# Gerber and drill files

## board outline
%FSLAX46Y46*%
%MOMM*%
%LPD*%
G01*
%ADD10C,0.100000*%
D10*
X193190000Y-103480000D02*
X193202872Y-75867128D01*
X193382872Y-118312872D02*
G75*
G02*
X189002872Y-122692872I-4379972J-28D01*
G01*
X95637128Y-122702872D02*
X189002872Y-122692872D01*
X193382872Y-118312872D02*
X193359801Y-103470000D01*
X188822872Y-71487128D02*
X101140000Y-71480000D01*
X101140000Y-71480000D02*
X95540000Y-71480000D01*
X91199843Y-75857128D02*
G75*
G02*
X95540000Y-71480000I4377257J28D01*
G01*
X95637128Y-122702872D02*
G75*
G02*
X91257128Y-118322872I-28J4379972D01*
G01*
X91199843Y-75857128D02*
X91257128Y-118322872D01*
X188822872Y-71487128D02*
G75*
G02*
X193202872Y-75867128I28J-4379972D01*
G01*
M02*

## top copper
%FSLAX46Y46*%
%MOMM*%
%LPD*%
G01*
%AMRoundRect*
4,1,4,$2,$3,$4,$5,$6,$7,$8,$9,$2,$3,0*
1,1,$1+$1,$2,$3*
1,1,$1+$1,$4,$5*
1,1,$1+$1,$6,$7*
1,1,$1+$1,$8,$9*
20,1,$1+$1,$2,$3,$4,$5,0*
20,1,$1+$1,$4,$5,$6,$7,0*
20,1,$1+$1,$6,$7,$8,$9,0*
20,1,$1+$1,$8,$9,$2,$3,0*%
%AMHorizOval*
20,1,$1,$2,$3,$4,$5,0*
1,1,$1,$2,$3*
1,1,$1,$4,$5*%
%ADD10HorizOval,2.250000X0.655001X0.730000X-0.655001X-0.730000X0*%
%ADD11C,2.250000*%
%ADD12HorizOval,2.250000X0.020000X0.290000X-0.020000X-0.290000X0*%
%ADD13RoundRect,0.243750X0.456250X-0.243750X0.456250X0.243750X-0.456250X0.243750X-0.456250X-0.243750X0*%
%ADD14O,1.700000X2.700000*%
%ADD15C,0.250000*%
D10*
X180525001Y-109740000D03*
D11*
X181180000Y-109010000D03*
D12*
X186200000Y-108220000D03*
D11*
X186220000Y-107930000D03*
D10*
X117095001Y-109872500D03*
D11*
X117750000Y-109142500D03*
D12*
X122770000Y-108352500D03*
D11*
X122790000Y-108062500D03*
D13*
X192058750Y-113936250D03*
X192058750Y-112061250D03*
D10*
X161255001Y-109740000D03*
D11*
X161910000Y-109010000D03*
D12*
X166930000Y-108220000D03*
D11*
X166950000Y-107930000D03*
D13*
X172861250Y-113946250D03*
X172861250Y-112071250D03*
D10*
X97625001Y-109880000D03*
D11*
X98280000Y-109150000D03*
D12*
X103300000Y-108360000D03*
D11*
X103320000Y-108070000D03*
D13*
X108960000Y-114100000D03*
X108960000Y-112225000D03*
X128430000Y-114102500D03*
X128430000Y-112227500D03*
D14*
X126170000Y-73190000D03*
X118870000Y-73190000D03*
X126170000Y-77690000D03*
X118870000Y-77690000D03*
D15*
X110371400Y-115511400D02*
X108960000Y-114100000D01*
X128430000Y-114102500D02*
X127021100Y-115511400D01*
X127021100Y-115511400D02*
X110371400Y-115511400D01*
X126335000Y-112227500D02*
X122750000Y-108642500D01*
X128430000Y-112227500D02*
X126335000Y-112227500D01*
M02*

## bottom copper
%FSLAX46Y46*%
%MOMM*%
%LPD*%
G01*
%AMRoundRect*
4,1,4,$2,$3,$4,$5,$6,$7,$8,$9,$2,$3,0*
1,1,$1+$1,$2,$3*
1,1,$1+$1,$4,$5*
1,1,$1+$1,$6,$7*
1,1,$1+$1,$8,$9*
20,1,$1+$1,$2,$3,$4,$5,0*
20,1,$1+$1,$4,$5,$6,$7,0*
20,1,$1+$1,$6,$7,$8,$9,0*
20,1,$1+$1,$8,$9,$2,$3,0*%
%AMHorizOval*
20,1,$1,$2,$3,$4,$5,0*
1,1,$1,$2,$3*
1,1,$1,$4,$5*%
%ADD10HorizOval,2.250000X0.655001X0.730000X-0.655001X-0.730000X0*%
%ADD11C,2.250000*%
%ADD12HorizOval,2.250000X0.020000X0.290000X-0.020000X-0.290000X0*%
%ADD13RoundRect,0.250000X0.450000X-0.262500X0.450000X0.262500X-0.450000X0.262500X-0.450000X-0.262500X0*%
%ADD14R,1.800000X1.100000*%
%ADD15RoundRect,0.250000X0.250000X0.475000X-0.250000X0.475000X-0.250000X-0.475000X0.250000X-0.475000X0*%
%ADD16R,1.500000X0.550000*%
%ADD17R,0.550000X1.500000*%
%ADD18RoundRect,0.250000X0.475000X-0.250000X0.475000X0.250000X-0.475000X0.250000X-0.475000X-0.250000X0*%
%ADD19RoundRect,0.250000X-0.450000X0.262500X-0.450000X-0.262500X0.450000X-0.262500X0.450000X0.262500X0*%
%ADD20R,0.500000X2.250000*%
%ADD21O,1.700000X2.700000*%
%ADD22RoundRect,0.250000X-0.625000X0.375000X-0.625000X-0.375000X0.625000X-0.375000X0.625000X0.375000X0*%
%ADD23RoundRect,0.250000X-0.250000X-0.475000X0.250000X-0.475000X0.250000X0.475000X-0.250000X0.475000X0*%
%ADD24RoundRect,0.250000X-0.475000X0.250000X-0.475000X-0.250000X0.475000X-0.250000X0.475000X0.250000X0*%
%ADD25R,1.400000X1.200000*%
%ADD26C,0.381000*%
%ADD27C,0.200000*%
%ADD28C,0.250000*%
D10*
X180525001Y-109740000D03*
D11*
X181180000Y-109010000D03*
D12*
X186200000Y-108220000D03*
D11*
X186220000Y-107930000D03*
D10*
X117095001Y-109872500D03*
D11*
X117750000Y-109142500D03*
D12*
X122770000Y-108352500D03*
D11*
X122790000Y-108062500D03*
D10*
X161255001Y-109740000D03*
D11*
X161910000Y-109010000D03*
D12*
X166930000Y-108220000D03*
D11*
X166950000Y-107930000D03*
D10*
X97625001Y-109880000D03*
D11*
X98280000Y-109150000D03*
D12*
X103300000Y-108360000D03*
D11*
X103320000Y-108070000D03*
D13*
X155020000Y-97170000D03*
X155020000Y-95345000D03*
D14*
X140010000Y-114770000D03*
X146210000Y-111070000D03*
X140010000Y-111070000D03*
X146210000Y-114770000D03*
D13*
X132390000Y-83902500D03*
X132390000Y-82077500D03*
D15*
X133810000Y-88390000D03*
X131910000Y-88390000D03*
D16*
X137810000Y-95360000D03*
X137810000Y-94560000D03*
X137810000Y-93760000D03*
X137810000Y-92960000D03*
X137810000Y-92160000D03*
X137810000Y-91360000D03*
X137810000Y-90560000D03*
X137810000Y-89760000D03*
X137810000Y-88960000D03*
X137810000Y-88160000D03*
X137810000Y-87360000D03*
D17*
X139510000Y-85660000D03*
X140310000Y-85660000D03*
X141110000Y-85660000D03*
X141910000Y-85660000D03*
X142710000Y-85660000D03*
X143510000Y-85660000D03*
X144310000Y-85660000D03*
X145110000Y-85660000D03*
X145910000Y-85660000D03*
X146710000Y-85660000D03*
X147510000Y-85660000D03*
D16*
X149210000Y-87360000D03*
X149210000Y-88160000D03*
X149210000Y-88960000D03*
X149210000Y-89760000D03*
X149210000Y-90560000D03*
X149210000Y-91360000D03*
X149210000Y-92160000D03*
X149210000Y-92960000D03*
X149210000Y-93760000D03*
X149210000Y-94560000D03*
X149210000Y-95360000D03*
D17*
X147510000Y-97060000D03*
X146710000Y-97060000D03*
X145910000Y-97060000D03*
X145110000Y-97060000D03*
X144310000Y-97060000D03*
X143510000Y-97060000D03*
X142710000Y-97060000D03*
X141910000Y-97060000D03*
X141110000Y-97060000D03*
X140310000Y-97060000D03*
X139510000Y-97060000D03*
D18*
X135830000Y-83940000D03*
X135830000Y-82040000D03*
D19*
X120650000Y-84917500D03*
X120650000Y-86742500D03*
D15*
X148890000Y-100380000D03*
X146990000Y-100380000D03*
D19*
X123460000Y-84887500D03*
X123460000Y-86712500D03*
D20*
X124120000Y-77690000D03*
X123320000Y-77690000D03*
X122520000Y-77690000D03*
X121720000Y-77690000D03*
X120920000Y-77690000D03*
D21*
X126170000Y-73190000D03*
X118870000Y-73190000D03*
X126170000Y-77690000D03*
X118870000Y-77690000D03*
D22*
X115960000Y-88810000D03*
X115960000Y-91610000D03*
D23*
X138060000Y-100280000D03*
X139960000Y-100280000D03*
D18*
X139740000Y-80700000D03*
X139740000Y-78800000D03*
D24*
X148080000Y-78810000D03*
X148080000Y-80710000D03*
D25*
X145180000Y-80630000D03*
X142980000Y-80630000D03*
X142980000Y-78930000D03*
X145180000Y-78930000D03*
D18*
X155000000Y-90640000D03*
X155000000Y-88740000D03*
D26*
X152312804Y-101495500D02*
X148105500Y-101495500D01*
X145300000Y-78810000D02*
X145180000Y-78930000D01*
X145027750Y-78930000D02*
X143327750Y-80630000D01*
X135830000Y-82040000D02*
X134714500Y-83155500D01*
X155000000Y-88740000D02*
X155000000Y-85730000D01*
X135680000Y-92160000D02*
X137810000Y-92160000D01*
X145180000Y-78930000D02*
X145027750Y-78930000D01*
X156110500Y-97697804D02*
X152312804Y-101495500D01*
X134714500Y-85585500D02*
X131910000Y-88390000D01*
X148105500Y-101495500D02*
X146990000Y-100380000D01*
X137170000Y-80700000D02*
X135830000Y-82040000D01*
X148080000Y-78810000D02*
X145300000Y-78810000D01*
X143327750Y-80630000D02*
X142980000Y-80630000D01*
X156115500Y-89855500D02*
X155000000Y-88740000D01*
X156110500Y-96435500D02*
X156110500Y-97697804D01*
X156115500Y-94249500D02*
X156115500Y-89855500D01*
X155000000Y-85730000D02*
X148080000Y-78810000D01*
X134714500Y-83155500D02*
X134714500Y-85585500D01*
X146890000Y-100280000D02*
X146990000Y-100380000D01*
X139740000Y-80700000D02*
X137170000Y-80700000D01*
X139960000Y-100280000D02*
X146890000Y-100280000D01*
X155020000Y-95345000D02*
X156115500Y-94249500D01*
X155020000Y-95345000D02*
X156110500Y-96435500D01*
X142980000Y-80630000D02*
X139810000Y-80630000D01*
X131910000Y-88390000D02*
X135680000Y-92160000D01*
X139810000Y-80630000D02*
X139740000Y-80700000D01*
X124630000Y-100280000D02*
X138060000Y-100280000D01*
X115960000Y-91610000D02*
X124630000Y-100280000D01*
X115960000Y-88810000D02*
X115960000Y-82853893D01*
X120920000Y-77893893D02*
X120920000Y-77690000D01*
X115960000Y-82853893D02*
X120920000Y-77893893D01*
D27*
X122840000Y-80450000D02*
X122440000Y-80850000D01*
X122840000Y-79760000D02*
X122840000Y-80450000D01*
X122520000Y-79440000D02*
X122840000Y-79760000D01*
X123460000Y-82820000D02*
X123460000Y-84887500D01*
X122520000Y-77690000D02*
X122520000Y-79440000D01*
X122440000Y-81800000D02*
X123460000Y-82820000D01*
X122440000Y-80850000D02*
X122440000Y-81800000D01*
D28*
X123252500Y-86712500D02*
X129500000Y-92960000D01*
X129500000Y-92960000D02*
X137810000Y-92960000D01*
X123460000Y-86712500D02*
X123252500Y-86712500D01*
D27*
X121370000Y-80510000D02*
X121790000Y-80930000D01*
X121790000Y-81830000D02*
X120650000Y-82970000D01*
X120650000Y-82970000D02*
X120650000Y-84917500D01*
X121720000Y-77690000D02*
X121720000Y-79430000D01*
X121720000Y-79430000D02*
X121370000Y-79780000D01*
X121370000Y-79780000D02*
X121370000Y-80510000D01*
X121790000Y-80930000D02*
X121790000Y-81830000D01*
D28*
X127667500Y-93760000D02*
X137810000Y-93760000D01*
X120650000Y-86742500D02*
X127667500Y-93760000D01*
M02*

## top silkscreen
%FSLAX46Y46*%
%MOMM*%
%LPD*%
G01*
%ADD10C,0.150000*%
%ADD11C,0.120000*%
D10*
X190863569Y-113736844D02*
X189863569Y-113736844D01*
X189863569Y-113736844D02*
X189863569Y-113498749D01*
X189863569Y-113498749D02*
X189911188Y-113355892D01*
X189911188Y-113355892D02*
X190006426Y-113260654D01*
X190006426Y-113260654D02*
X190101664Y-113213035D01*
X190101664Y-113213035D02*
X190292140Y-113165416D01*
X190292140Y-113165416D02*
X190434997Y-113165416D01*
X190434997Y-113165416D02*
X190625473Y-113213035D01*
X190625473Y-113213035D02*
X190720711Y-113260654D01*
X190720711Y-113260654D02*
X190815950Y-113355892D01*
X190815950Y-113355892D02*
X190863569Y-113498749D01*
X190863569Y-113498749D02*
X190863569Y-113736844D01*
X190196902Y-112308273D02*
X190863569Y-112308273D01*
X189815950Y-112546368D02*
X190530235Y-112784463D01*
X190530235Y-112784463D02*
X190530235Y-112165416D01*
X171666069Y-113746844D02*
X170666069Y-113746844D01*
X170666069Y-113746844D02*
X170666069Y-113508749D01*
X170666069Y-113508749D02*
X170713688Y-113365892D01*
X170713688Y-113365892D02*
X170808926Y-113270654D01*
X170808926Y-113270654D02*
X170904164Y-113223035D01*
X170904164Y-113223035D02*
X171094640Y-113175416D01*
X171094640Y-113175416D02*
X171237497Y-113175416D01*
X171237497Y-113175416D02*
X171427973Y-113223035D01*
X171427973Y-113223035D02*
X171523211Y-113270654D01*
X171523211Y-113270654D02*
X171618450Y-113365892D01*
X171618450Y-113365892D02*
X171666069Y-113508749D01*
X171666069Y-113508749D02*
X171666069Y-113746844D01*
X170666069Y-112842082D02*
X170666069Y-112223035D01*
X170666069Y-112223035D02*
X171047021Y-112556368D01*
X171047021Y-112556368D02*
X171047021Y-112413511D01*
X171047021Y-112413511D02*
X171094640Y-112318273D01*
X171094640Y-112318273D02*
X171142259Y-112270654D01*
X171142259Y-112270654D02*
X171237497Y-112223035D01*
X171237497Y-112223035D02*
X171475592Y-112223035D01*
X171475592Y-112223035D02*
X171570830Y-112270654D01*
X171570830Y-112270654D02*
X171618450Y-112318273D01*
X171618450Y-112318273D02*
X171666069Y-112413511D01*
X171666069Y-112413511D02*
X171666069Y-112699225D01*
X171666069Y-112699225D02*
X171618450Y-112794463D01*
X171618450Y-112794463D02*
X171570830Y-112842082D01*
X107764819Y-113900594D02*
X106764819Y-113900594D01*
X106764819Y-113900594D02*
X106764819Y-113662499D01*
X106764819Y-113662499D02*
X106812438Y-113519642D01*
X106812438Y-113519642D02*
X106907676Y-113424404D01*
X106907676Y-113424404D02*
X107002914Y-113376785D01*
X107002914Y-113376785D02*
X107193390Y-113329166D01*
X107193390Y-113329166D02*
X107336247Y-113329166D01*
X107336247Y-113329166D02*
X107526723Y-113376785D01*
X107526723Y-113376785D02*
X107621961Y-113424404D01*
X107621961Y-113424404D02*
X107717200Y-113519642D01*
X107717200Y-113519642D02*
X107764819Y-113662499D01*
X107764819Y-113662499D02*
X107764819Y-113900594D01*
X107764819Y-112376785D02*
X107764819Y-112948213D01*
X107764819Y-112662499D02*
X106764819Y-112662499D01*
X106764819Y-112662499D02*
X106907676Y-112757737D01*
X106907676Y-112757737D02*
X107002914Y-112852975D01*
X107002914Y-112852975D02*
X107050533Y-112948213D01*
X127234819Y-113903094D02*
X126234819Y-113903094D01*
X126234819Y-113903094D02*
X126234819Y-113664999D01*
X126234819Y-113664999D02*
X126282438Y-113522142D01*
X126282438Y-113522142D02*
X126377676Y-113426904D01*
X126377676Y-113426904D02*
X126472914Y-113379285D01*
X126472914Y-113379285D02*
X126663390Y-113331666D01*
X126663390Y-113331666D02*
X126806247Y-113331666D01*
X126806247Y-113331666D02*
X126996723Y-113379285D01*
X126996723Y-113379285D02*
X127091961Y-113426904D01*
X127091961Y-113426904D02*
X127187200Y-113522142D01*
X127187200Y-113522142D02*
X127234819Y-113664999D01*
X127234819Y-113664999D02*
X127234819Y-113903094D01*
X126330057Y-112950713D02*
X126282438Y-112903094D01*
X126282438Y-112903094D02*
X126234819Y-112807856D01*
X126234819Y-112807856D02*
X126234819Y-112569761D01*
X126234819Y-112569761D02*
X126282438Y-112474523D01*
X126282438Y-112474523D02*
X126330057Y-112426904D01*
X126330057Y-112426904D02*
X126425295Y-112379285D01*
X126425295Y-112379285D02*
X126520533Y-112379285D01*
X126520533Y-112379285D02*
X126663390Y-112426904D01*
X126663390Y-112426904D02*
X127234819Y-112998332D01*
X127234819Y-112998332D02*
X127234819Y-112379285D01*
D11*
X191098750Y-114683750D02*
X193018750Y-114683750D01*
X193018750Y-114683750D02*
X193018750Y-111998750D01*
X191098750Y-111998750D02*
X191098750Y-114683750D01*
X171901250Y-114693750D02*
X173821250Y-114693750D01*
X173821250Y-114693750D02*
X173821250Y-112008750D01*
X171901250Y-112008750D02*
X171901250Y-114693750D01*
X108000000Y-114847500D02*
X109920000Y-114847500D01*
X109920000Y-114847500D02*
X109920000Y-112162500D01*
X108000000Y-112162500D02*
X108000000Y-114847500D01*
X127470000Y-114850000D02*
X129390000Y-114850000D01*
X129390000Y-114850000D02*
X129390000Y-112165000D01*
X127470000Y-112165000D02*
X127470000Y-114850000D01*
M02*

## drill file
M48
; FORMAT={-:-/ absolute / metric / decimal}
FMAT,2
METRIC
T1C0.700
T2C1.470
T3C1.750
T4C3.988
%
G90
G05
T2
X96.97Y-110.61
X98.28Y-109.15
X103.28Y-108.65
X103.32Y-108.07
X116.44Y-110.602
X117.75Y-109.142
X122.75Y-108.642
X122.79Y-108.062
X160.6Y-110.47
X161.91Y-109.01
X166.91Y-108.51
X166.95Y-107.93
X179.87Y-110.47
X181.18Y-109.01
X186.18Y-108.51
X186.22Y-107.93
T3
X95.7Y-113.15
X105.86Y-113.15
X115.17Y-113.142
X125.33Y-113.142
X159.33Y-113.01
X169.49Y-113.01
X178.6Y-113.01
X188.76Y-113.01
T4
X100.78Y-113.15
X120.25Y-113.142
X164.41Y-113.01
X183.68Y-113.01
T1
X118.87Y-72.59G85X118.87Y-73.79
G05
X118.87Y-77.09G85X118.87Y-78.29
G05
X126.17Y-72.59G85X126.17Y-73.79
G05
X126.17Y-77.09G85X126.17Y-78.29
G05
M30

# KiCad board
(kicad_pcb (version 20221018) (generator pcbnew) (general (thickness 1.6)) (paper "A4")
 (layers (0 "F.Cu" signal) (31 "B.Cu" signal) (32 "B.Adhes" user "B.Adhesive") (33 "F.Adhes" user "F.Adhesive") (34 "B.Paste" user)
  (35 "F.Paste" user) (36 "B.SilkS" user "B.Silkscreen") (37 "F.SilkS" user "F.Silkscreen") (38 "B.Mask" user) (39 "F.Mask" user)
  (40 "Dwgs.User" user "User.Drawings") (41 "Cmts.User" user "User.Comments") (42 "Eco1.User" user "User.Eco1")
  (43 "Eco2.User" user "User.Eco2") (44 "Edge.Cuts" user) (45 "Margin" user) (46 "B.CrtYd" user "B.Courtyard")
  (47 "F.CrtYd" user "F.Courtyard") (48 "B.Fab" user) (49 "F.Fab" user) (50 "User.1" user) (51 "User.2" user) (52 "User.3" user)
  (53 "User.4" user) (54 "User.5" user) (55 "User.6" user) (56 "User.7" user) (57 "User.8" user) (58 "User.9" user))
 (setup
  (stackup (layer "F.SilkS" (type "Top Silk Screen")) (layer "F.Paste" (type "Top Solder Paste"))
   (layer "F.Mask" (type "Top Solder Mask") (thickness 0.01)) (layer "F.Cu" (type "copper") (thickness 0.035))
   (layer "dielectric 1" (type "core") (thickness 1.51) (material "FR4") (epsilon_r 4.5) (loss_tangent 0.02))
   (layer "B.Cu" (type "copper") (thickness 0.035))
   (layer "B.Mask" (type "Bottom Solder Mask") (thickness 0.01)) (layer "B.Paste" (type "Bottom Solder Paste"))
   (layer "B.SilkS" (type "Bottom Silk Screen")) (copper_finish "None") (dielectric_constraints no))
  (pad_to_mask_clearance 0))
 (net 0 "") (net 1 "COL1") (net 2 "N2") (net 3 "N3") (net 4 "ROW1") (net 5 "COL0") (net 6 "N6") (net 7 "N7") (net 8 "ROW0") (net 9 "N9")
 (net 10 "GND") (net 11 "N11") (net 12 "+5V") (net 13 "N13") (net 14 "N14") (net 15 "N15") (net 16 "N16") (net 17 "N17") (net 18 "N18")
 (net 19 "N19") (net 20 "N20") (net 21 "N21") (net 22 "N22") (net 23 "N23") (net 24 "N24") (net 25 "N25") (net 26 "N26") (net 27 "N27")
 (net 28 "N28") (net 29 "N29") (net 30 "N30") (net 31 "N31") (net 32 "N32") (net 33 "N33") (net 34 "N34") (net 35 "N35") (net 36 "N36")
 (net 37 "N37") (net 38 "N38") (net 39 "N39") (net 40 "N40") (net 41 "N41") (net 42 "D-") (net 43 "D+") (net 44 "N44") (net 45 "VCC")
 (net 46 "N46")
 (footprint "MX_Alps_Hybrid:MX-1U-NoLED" (layer "F.Cu") (at 183.68 113.01)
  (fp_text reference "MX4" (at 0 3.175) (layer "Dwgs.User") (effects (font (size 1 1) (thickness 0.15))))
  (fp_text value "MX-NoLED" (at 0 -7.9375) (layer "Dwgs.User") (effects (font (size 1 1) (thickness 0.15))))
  (pad "" np_thru_hole circle (at -5.08 0 48.0996) (size 1.75 1.75) (drill 1.75) (layers "*.Cu" "*.Mask"))
  (pad "" np_thru_hole circle (at 0 0) (size 3.9878 3.9878) (drill 3.9878) (layers "*.Cu" "*.Mask"))
  (pad "" np_thru_hole circle (at 5.08 0 48.0996) (size 1.75 1.75) (drill 1.75) (layers "*.Cu" "*.Mask"))
  (pad "1" thru_hole oval (at -3.81 -2.54 48.0996) (size 4.211556 2.25) (drill 1.47 (offset 0.980778 0)) (layers "*.Cu" "B.Mask")
   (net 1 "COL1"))
  (pad "1" thru_hole circle (at -2.5 -4) (size 2.25 2.25) (drill 1.47) (layers "*.Cu" "B.Mask") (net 1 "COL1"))
  (pad "2" thru_hole oval (at 2.5 -4.5 86.0548) (size 2.831378 2.25) (drill 1.47 (offset 0.290689 0)) (layers "*.Cu" "B.Mask") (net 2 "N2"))
  (pad "2" thru_hole circle (at 2.54 -5.08) (size 2.25 2.25) (drill 1.47) (layers "*.Cu" "B.Mask") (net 2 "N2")))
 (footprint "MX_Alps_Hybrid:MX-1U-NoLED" (layer "F.Cu") (at 120.25 113.1425)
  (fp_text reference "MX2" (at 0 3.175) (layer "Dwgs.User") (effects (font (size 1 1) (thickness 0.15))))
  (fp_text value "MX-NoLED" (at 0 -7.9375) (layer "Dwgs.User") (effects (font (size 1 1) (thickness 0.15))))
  (pad "" np_thru_hole circle (at -5.08 0 48.0996) (size 1.75 1.75) (drill 1.75) (layers "*.Cu" "*.Mask"))
  (pad "" np_thru_hole circle (at 0 0) (size 3.9878 3.9878) (drill 3.9878) (layers "*.Cu" "*.Mask"))
  (pad "" np_thru_hole circle (at 5.08 0 48.0996) (size 1.75 1.75) (drill 1.75) (layers "*.Cu" "*.Mask"))
  (pad "1" thru_hole oval (at -3.81 -2.54 48.0996) (size 4.211556 2.25) (drill 1.47 (offset 0.980778 0)) (layers "*.Cu" "B.Mask")
   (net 1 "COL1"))
  (pad "1" thru_hole circle (at -2.5 -4) (size 2.25 2.25) (drill 1.47) (layers "*.Cu" "B.Mask") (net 1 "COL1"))
  (pad "2" thru_hole oval (at 2.5 -4.5 86.0548) (size 2.831378 2.25) (drill 1.47 (offset 0.290689 0)) (layers "*.Cu" "B.Mask") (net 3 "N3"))
  (pad "2" thru_hole circle (at 2.54 -5.08) (size 2.25 2.25) (drill 1.47) (layers "*.Cu" "B.Mask") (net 3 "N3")))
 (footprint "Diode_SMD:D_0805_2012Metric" (layer "F.Cu") (at 192.05875 112.99875 90)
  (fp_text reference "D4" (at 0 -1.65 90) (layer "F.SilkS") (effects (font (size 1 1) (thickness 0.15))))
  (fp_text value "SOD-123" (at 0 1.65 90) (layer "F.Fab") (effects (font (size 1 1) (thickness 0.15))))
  (fp_line (start -1.685 -0.96) (end -1.685 0.96) (stroke (width 0.12) (type solid)) (layer "F.SilkS"))
  (fp_line (start -1.685 0.96) (end 1 0.96) (stroke (width 0.12) (type solid)) (layer "F.SilkS"))
  (fp_line (start 1 -0.96) (end -1.685 -0.96) (stroke (width 0.12) (type solid)) (layer "F.SilkS"))
  (pad "1" smd roundrect (at -0.9375 0 90) (size 0.975 1.4) (layers "F.Cu" "F.Paste" "F.Mask") (roundrect_rratio 0.25) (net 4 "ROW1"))
  (pad "2" smd roundrect (at 0.9375 0 90) (size 0.975 1.4) (layers "F.Cu" "F.Paste" "F.Mask") (roundrect_rratio 0.25) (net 2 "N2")))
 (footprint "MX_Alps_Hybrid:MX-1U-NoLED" (layer "F.Cu") (at 164.41 113.01)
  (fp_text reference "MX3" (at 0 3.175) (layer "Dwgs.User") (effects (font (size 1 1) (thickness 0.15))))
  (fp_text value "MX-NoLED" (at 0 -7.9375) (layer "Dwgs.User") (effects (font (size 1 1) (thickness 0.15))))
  (pad "" np_thru_hole circle (at -5.08 0 48.0996) (size 1.75 1.75) (drill 1.75) (layers "*.Cu" "*.Mask"))
  (pad "" np_thru_hole circle (at 0 0) (size 3.9878 3.9878) (drill 3.9878) (layers "*.Cu" "*.Mask"))
  (pad "" np_thru_hole circle (at 5.08 0 48.0996) (size 1.75 1.75) (drill 1.75) (layers "*.Cu" "*.Mask"))
  (pad "1" thru_hole oval (at -3.81 -2.54 48.0996) (size 4.211556 2.25) (drill 1.47 (offset 0.980778 0)) (layers "*.Cu" "B.Mask")
   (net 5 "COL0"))
  (pad "1" thru_hole circle (at -2.5 -4) (size 2.25 2.25) (drill 1.47) (layers "*.Cu" "B.Mask") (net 5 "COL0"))
  (pad "2" thru_hole oval (at 2.5 -4.5 86.0548) (size 2.831378 2.25) (drill 1.47 (offset 0.290689 0)) (layers "*.Cu" "B.Mask") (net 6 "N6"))
  (pad "2" thru_hole circle (at 2.54 -5.08) (size 2.25 2.25) (drill 1.47) (layers "*.Cu" "B.Mask") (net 6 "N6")))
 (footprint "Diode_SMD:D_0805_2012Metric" (layer "F.Cu") (at 172.86125 113.00875 90)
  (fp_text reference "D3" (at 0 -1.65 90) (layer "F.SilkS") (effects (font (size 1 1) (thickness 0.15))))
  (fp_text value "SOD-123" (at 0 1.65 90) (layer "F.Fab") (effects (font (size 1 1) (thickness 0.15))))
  (fp_line (start -1.685 -0.96) (end -1.685 0.96) (stroke (width 0.12) (type solid)) (layer "F.SilkS"))
  (fp_line (start -1.685 0.96) (end 1 0.96) (stroke (width 0.12) (type solid)) (layer "F.SilkS"))
  (fp_line (start 1 -0.96) (end -1.685 -0.96) (stroke (width 0.12) (type solid)) (layer "F.SilkS"))
  (pad "1" smd roundrect (at -0.9375 0 90) (size 0.975 1.4) (layers "F.Cu" "F.Paste" "F.Mask") (roundrect_rratio 0.25) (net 4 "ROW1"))
  (pad "2" smd roundrect (at 0.9375 0 90) (size 0.975 1.4) (layers "F.Cu" "F.Paste" "F.Mask") (roundrect_rratio 0.25) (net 6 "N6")))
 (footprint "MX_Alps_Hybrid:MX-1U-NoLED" (layer "F.Cu") (at 100.78 113.15)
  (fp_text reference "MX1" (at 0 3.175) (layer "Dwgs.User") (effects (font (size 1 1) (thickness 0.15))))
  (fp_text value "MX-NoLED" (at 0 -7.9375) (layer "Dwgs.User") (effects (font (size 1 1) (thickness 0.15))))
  (pad "" np_thru_hole circle (at -5.08 0 48.0996) (size 1.75 1.75) (drill 1.75) (layers "*.Cu" "*.Mask"))
  (pad "" np_thru_hole circle (at 0 0) (size 3.9878 3.9878) (drill 3.9878) (layers "*.Cu" "*.Mask"))
  (pad "" np_thru_hole circle (at 5.08 0 48.0996) (size 1.75 1.75) (drill 1.75) (layers "*.Cu" "*.Mask"))
  (pad "1" thru_hole oval (at -3.81 -2.54 48.0996) (size 4.211556 2.25) (drill 1.47 (offset 0.980778 0)) (layers "*.Cu" "B.Mask")
   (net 5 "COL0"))
  (pad "1" thru_hole circle (at -2.5 -4) (size 2.25 2.25) (drill 1.47) (layers "*.Cu" "B.Mask") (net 5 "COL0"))
  (pad "2" thru_hole oval (at 2.5 -4.5 86.0548) (size 2.831378 2.25) (drill 1.47 (offset 0.290689 0)) (layers "*.Cu" "B.Mask") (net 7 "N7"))
  (pad "2" thru_hole circle (at 2.54 -5.08) (size 2.25 2.25) (drill 1.47) (layers "*.Cu" "B.Mask") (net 7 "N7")))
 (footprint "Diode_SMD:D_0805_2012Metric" (layer "F.Cu") (at 108.96 113.1625 90)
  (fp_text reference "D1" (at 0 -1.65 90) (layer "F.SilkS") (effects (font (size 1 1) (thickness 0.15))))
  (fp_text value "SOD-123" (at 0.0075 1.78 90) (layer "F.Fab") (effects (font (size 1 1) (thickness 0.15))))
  (fp_line (start -1.685 -0.96) (end -1.685 0.96) (stroke (width 0.12) (type solid)) (layer "F.SilkS"))
  (fp_line (start -1.685 0.96) (end 1 0.96) (stroke (width 0.12) (type solid)) (layer "F.SilkS"))
  (fp_line (start 1 -0.96) (end -1.685 -0.96) (stroke (width 0.12) (type solid)) (layer "F.SilkS"))
  (pad "1" smd roundrect (at -0.9375 0 90) (size 0.975 1.4) (layers "F.Cu" "F.Paste" "F.Mask") (roundrect_rratio 0.25) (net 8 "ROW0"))
  (pad "2" smd roundrect (at 0.9375 0 90) (size 0.975 1.4) (layers "F.Cu" "F.Paste" "F.Mask") (roundrect_rratio 0.25) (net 7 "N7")))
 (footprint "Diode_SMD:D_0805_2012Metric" (layer "F.Cu") (at 128.43 113.165 90)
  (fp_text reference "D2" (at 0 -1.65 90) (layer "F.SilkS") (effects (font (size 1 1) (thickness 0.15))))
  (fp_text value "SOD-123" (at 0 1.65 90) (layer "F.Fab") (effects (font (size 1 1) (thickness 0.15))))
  (fp_line (start -1.685 -0.96) (end -1.685 0.96) (stroke (width 0.12) (type solid)) (layer "F.SilkS"))
  (fp_line (start -1.685 0.96) (end 1 0.96) (stroke (width 0.12) (type solid)) (layer "F.SilkS"))
  (fp_line (start 1 -0.96) (end -1.685 -0.96) (stroke (width 0.12) (type solid)) (layer "F.SilkS"))
  (pad "1" smd roundrect (at -0.9375 0 90) (size 0.975 1.4) (layers "F.Cu" "F.Paste" "F.Mask") (roundrect_rratio 0.25) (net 8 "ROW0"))
  (pad "2" smd roundrect (at 0.9375 0 90) (size 0.975 1.4) (layers "F.Cu" "F.Paste" "F.Mask") (roundrect_rratio 0.25) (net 3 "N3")))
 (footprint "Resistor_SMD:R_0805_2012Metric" (layer "B.Cu") (at 155.02 96.2575 90)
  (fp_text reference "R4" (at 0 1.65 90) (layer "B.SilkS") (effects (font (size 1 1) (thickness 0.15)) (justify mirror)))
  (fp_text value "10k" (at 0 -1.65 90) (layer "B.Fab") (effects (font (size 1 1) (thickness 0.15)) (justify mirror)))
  (pad "1" smd roundrect (at -0.9125 0 90) (size 1.025 1.4) (layers "B.Cu" "B.Paste" "B.Mask") (roundrect_rratio 0.243902) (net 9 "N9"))
  (pad "2" smd roundrect (at 0.9125 0 90) (size 1.025 1.4) (layers "B.Cu" "B.Paste" "B.Mask") (roundrect_rratio 0.243902) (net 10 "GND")))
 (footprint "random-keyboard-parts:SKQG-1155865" (layer "B.Cu") (at 143.11 112.92 180)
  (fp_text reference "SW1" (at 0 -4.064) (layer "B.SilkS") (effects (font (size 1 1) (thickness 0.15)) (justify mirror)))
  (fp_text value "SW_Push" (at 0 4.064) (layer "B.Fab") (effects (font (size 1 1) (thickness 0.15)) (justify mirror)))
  (pad "1" smd rect (at 3.1 -1.85 180) (size 1.8 1.1) (layers "B.Cu" "B.Paste" "B.Mask") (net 10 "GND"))
  (pad "2" smd rect (at -3.1 1.85 180) (size 1.8 1.1) (layers "B.Cu" "B.Paste" "B.Mask") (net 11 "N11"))
  (pad "3" smd rect (at 3.1 1.85 180) (size 1.8 1.1) (layers "B.Cu" "B.Paste" "B.Mask"))
  (pad "4" smd rect (at -3.1 -1.85 180) (size 1.8 1.1) (layers "B.Cu" "B.Paste" "B.Mask")))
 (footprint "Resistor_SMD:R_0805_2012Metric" (layer "B.Cu") (at 132.39 82.99 90)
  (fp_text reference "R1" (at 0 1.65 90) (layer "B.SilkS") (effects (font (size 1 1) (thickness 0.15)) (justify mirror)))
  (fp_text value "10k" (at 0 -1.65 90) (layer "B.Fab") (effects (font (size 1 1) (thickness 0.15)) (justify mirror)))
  (pad "1" smd roundrect (at -0.9125 0 90) (size 1.025 1.4) (layers "B.Cu" "B.Paste" "B.Mask") (roundrect_rratio 0.243902) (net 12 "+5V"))
  (pad "2" smd roundrect (at 0.9125 0 90) (size 1.025 1.4) (layers "B.Cu" "B.Paste" "B.Mask") (roundrect_rratio 0.243902) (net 11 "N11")))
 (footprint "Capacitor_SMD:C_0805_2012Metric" (layer "B.Cu") (at 132.86 88.39 180)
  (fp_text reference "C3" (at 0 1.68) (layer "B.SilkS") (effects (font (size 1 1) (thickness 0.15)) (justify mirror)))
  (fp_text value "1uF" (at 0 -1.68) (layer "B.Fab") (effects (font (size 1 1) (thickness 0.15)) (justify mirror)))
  (pad "1" smd roundrect (at -0.95 0 180) (size 1 1.45) (layers "B.Cu" "B.Paste" "B.Mask") (roundrect_rratio 0.25) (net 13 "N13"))
  (pad "2" smd roundrect (at 0.95 0 180) (size 1 1.45) (layers "B.Cu" "B.Paste" "B.Mask") (roundrect_rratio 0.25) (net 10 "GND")))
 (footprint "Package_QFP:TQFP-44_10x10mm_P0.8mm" (layer "B.Cu") (at 143.51 91.36)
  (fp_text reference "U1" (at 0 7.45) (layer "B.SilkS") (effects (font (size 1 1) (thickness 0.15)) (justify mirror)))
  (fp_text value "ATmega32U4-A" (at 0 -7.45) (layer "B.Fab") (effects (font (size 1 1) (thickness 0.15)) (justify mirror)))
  (pad "1" smd rect (at -5.7 4) (size 1.5 0.55) (layers "B.Cu" "B.Paste" "B.Mask") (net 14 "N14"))
  (pad "2" smd rect (at -5.7 3.2) (size 1.5 0.55) (layers "B.Cu" "B.Paste" "B.Mask") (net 12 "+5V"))
  (pad "3" smd rect (at -5.7 2.4) (size 1.5 0.55) (layers "B.Cu" "B.Paste" "B.Mask") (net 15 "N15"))
  (pad "4" smd rect (at -5.7 1.6) (size 1.5 0.55) (layers "B.Cu" "B.Paste" "B.Mask") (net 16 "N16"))
  (pad "5" smd rect (at -5.7 0.8) (size 1.5 0.55) (layers "B.Cu" "B.Paste" "B.Mask") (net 10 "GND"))
  (pad "6" smd rect (at -5.7 0) (size 1.5 0.55) (layers "B.Cu" "B.Paste" "B.Mask") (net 13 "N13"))
  (pad "7" smd rect (at -5.7 -0.8) (size 1.5 0.55) (layers "B.Cu" "B.Paste" "B.Mask") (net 12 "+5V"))
  (pad "8" smd rect (at -5.7 -1.6) (size 1.5 0.55) (layers "B.Cu" "B.Paste" "B.Mask") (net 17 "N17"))
  (pad "9" smd rect (at -5.7 -2.4) (size 1.5 0.55) (layers "B.Cu" "B.Paste" "B.Mask") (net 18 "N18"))
  (pad "10" smd rect (at -5.7 -3.2) (size 1.5 0.55) (layers "B.Cu" "B.Paste" "B.Mask") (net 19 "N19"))
  (pad "11" smd rect (at -5.7 -4) (size 1.5 0.55) (layers "B.Cu" "B.Paste" "B.Mask") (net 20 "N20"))
  (pad "12" smd rect (at -4 -5.7 270) (size 1.5 0.55) (layers "B.Cu" "B.Paste" "B.Mask") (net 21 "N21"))
  (pad "13" smd rect (at -3.2 -5.7 270) (size 1.5 0.55) (layers "B.Cu" "B.Paste" "B.Mask") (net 11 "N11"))
  (pad "14" smd rect (at -2.4 -5.7 270) (size 1.5 0.55) (layers "B.Cu" "B.Paste" "B.Mask") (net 12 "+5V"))
  (pad "15" smd rect (at -1.6 -5.7 270) (size 1.5 0.55) (layers "B.Cu" "B.Paste" "B.Mask") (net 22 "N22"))
  (pad "16" smd rect (at -0.8 -5.7 270) (size 1.5 0.55) (layers "B.Cu" "B.Paste" "B.Mask") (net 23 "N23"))
  (pad "17" smd rect (at 0 -5.7 270) (size 1.5 0.55) (layers "B.Cu" "B.Paste" "B.Mask") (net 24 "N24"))
  (pad "18" smd rect (at 0.8 -5.7 270) (size 1.5 0.55) (layers "B.Cu" "B.Paste" "B.Mask") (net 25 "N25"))
  (pad "19" smd rect (at 1.6 -5.7 270) (size 1.5 0.55) (layers "B.Cu" "B.Paste" "B.Mask") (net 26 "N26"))
  (pad "20" smd rect (at 2.4 -5.7 270) (size 1.5 0.55) (layers "B.Cu" "B.Paste" "B.Mask") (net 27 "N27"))
  (pad "21" smd rect (at 3.2 -5.7 270) (size 1.5 0.55) (layers "B.Cu" "B.Paste" "B.Mask") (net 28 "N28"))
  (pad "22" smd rect (at 4 -5.7 270) (size 1.5 0.55) (layers "B.Cu" "B.Paste" "B.Mask") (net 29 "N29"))
  (pad "23" smd rect (at 5.7 -4) (size 1.5 0.55) (layers "B.Cu" "B.Paste" "B.Mask") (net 22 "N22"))
  (pad "24" smd rect (at 5.7 -3.2) (size 1.5 0.55) (layers "B.Cu" "B.Paste" "B.Mask") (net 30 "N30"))
  (pad "25" smd rect (at 5.7 -2.4) (size 1.5 0.55) (layers "B.Cu" "B.Paste" "B.Mask") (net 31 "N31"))
  (pad "26" smd rect (at 5.7 -1.6) (size 1.5 0.55) (layers "B.Cu" "B.Paste" "B.Mask") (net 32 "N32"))
  (pad "27" smd rect (at 5.7 -0.8) (size 1.5 0.55) (layers "B.Cu" "B.Paste" "B.Mask") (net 8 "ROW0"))
  (pad "28" smd rect (at 5.7 0) (size 1.5 0.55) (layers "B.Cu" "B.Paste" "B.Mask") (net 1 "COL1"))
  (pad "29" smd rect (at 5.7 0.8) (size 1.5 0.55) (layers "B.Cu" "B.Paste" "B.Mask") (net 5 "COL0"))
  (pad "30" smd rect (at 5.7 1.6) (size 1.5 0.55) (layers "B.Cu" "B.Paste" "B.Mask") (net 4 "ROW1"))
  (pad "31" smd rect (at 5.7 2.4) (size 1.5 0.55) (layers "B.Cu" "B.Paste" "B.Mask") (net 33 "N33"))
  (pad "32" smd rect (at 5.7 3.2) (size 1.5 0.55) (layers "B.Cu" "B.Paste" "B.Mask") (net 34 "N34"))
  (pad "33" smd rect (at 5.7 4) (size 1.5 0.55) (layers "B.Cu" "B.Paste" "B.Mask") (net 9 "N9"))
  (pad "34" smd rect (at 4 5.7 270) (size 1.5 0.55) (layers "B.Cu" "B.Paste" "B.Mask") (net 12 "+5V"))
  (pad "35" smd rect (at 3.2 5.7 270) (size 1.5 0.55) (layers "B.Cu" "B.Paste" "B.Mask") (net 22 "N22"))
  (pad "36" smd rect (at 2.4 5.7 270) (size 1.5 0.55) (layers "B.Cu" "B.Paste" "B.Mask") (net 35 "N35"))
  (pad "37" smd rect (at 1.6 5.7 270) (size 1.5 0.55) (layers "B.Cu" "B.Paste" "B.Mask") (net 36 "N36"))
  (pad "38" smd rect (at 0.8 5.7 270) (size 1.5 0.55) (layers "B.Cu" "B.Paste" "B.Mask") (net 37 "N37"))
  (pad "39" smd rect (at 0 5.7 270) (size 1.5 0.55) (layers "B.Cu" "B.Paste" "B.Mask") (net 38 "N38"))
  (pad "40" smd rect (at -0.8 5.7 270) (size 1.5 0.55) (layers "B.Cu" "B.Paste" "B.Mask") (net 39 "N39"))
  (pad "41" smd rect (at -1.6 5.7 270) (size 1.5 0.55) (layers "B.Cu" "B.Paste" "B.Mask") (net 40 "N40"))
  (pad "42" smd rect (at -2.4 5.7 270) (size 1.5 0.55) (layers "B.Cu" "B.Paste" "B.Mask") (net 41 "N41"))
  (pad "43" smd rect (at -3.2 5.7 270) (size 1.5 0.55) (layers "B.Cu" "B.Paste" "B.Mask") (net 22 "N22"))
  (pad "44" smd rect (at -4 5.7 270) (size 1.5 0.55) (layers "B.Cu" "B.Paste" "B.Mask") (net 30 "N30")))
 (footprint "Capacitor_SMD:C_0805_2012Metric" (layer "B.Cu") (at 135.83 82.99 90)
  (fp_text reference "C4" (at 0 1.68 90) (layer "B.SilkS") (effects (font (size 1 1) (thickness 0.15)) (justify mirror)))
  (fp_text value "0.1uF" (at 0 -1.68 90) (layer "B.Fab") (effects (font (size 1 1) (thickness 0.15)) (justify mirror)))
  (pad "1" smd roundrect (at -0.95 0 90) (size 1 1.45) (layers "B.Cu" "B.Paste" "B.Mask") (roundrect_rratio 0.25) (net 12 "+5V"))
  (pad "2" smd roundrect (at 0.95 0 90) (size 1 1.45) (layers "B.Cu" "B.Paste" "B.Mask") (roundrect_rratio 0.25) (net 10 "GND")))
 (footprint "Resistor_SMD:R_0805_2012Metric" (layer "B.Cu") (at 120.65 85.83 -90)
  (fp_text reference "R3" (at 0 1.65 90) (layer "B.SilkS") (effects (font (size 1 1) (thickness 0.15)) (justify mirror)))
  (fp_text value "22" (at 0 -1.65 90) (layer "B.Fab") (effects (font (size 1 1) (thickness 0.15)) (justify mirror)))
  (pad "1" smd roundrect (at -0.9125 0 270) (size 1.025 1.4) (layers "B.Cu" "B.Paste" "B.Mask") (roundrect_rratio 0.243902) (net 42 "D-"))
  (pad "2" smd roundrect (at 0.9125 0 270) (size 1.025 1.4) (layers "B.Cu" "B.Paste" "B.Mask") (roundrect_rratio 0.243902) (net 15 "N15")))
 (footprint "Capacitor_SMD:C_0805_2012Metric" (layer "B.Cu") (at 147.94 100.38 180)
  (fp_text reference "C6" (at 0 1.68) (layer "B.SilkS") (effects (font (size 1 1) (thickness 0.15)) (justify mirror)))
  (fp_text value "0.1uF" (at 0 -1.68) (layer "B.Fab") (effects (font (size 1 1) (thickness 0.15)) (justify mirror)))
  (pad "1" smd roundrect (at -0.95 0 180) (size 1 1.45) (layers "B.Cu" "B.Paste" "B.Mask") (roundrect_rratio 0.25) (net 12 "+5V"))
  (pad "2" smd roundrect (at 0.95 0 180) (size 1 1.45) (layers "B.Cu" "B.Paste" "B.Mask") (roundrect_rratio 0.25) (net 10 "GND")))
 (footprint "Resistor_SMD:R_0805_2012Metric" (layer "B.Cu") (at 123.46 85.8 -90)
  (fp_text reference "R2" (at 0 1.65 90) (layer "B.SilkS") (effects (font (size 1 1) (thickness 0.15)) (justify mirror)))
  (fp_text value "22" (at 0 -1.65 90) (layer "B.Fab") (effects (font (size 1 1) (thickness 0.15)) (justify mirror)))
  (pad "1" smd roundrect (at -0.9125 0 270) (size 1.025 1.4) (layers "B.Cu" "B.Paste" "B.Mask") (roundrect_rratio 0.243902) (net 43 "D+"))
  (pad "2" smd roundrect (at 0.9125 0 270) (size 1.025 1.4) (layers "B.Cu" "B.Paste" "B.Mask") (roundrect_rratio 0.243902) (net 16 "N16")))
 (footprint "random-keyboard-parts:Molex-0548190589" (layer "B.Cu") (at 122.52 73.19 -90)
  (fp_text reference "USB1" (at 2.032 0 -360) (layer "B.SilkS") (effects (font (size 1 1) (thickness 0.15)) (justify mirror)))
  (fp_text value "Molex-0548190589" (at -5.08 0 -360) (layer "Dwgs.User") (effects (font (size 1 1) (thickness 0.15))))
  (pad "1" smd rect (at 4.5 -1.6 270) (size 2.25 0.5) (layers "B.Cu" "B.Paste" "B.Mask") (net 10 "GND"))
  (pad "2" smd rect (at 4.5 -0.8 270) (size 2.25 0.5) (layers "B.Cu" "B.Paste" "B.Mask") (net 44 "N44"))
  (pad "3" smd rect (at 4.5 0 270) (size 2.25 0.5) (layers "B.Cu" "B.Paste" "B.Mask") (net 43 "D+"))
  (pad "4" smd rect (at 4.5 0.8 270) (size 2.25 0.5) (layers "B.Cu" "B.Paste" "B.Mask") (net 42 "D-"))
  (pad "5" smd rect (at 4.5 1.6 270) (size 2.25 0.5) (layers "B.Cu" "B.Paste" "B.Mask") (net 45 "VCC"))
  (pad "6" thru_hole oval (at 0 -3.65 270) (size 2.7 1.7) (drill oval 1.9 0.7) (layers "*.Cu" "*.Mask") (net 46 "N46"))
  (pad "6" thru_hole oval (at 0 3.65 270) (size 2.7 1.7) (drill oval 1.9 0.7) (layers "*.Cu" "*.Mask") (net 46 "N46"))
  (pad "6" thru_hole oval (at 4.5 -3.65 270) (size 2.7 1.7) (drill oval 1.9 0.7) (layers "*.Cu" "*.Mask") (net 46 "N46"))
  (pad "6" thru_hole oval (at 4.5 3.65 270) (size 2.7 1.7) (drill oval 1.9 0.7) (layers "*.Cu" "*.Mask") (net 46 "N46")))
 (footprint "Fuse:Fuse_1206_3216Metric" (layer "B.Cu") (at 115.96 90.21 -90)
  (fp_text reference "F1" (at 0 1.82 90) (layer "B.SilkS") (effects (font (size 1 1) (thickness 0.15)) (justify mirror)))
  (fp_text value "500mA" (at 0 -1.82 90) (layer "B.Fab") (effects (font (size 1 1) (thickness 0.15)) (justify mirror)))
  (pad "1" smd roundrect (at -1.4 0 270) (size 1.25 1.75) (layers "B.Cu" "B.Paste" "B.Mask") (roundrect_rratio 0.2) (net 45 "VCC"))
  (pad "2" smd roundrect (at 1.4 0 270) (size 1.25 1.75) (layers "B.Cu" "B.Paste" "B.Mask") (roundrect_rratio 0.2) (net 12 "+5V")))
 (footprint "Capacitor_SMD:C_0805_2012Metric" (layer "B.Cu") (at 139.01 100.28)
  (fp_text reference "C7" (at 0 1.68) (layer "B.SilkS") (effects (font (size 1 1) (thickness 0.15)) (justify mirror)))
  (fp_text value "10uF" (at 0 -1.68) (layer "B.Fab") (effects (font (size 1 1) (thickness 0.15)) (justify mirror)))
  (pad "1" smd roundrect (at -0.95 0) (size 1 1.45) (layers "B.Cu" "B.Paste" "B.Mask") (roundrect_rratio 0.25) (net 12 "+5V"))
  (pad "2" smd roundrect (at 0.95 0) (size 1 1.45) (layers "B.Cu" "B.Paste" "B.Mask") (roundrect_rratio 0.25) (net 10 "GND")))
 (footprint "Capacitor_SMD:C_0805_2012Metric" (layer "B.Cu") (at 139.74 79.75 90)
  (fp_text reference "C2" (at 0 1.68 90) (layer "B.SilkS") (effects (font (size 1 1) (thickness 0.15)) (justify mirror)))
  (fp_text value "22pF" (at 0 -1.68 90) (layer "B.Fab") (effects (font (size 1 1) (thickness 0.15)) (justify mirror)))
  (pad "1" smd roundrect (at -0.95 0 90) (size 1 1.45) (layers "B.Cu" "B.Paste" "B.Mask") (roundrect_rratio 0.25) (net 10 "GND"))
  (pad "2" smd roundrect (at 0.95 0 90) (size 1 1.45) (layers "B.Cu" "B.Paste" "B.Mask") (roundrect_rratio 0.25) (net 23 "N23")))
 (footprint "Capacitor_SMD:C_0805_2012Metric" (layer "B.Cu") (at 148.08 79.76 -90)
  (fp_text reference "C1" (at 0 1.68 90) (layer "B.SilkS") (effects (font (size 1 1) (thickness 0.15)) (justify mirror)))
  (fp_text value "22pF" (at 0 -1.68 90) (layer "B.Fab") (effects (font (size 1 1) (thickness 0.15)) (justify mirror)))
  (pad "1" smd roundrect (at -0.95 0 270) (size 1 1.45) (layers "B.Cu" "B.Paste" "B.Mask") (roundrect_rratio 0.25) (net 10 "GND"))
  (pad "2" smd roundrect (at 0.95 0 270) (size 1 1.45) (layers "B.Cu" "B.Paste" "B.Mask") (roundrect_rratio 0.25) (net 24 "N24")))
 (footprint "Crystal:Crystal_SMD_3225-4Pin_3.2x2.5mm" (layer "B.Cu") (at 144.08 79.78 180)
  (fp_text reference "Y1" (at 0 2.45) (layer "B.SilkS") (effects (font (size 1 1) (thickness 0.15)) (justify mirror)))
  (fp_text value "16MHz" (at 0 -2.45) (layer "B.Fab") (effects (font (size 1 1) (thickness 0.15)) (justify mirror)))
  (pad "1" smd rect (at -1.1 -0.85 180) (size 1.4 1.2) (layers "B.Cu" "B.Paste" "B.Mask") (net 24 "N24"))
  (pad "2" smd rect (at 1.1 -0.85 180) (size 1.4 1.2) (layers "B.Cu" "B.Paste" "B.Mask") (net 10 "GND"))
  (pad "3" smd rect (at 1.1 0.85 180) (size 1.4 1.2) (layers "B.Cu" "B.Paste" "B.Mask") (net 23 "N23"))
  (pad "4" smd rect (at -1.1 0.85 180) (size 1.4 1.2) (layers "B.Cu" "B.Paste" "B.Mask") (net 10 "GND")))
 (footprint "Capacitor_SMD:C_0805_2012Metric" (layer "B.Cu") (at 155 89.69 90)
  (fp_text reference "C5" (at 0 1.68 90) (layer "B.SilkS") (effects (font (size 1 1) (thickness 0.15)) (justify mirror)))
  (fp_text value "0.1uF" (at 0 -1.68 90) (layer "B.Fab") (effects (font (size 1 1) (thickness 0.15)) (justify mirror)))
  (pad "1" smd roundrect (at -0.95 0 90) (size 1 1.45) (layers "B.Cu" "B.Paste" "B.Mask") (roundrect_rratio 0.25) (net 12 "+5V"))
  (pad "2" smd roundrect (at 0.95 0 90) (size 1 1.45) (layers "B.Cu" "B.Paste" "B.Mask") (roundrect_rratio 0.25) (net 10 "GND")))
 (gr_line (start 193.19 103.48) (end 193.202872 75.867128) (stroke (width 0.1) (type default)) (layer "Edge.Cuts"))
 (gr_arc (start 193.382872 118.312872) (mid 192.1 121.41) (end 189.002872 122.692872) (stroke (width 0.1) (type default))
  (layer "Edge.Cuts"))
 (gr_line (start 95.637128 122.702872) (end 189.002872 122.692872) (stroke (width 0.1) (type default)) (layer "Edge.Cuts"))
 (gr_line (start 193.382872 118.312872) (end 193.359801 103.47) (stroke (width 0.1) (type default)) (layer "Edge.Cuts"))
 (gr_line (start 188.822872 71.487128) (end 101.14 71.48) (stroke (width 0.1) (type default)) (layer "Edge.Cuts"))
 (gr_line (start 101.14 71.48) (end 95.54 71.48) (stroke (width 0.1) (type default)) (layer "Edge.Cuts"))
 (gr_arc (start 91.199843 75.857128) (mid 92.468821 72.775074) (end 95.54 71.48) (stroke (width 0.1) (type default)) (layer "Edge.Cuts"))
 (gr_arc (start 95.637128 122.702872) (mid 92.54 121.42) (end 91.257128 118.322872) (stroke (width 0.1) (type default)) (layer "Edge.Cuts"))
 (gr_line (start 91.199843 75.857128) (end 91.257128 118.322872) (stroke (width 0.1) (type default)) (layer "Edge.Cuts"))
 (gr_arc (start 188.822872 71.487128) (mid 191.92 72.77) (end 193.202872 75.867128) (stroke (width 0.1) (type default)) (layer "Edge.Cuts"))
 (segment (start 152.312804 101.4955) (end 148.1055 101.4955) (width 0.381) (layer "B.Cu") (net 10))
 (segment (start 145.3 78.81) (end 145.18 78.93) (width 0.381) (layer "B.Cu") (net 10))
 (segment (start 145.02775 78.93) (end 143.32775 80.63) (width 0.381) (layer "B.Cu") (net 10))
 (segment (start 135.83 82.04) (end 134.7145 83.1555) (width 0.381) (layer "B.Cu") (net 10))
 (segment (start 155 88.74) (end 155 85.73) (width 0.381) (layer "B.Cu") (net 10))
 (segment (start 135.68 92.16) (end 137.81 92.16) (width 0.381) (layer "B.Cu") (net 10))
 (segment (start 145.18 78.93) (end 145.02775 78.93) (width 0.381) (layer "B.Cu") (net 10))
 (segment (start 156.1105 97.697804) (end 152.312804 101.4955) (width 0.381) (layer "B.Cu") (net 10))
 (segment (start 134.7145 85.5855) (end 131.91 88.39) (width 0.381) (layer "B.Cu") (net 10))
 (segment (start 148.1055 101.4955) (end 146.99 100.38) (width 0.381) (layer "B.Cu") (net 10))
 (segment (start 137.17 80.7) (end 135.83 82.04) (width 0.381) (layer "B.Cu") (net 10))
 (segment (start 148.08 78.81) (end 145.3 78.81) (width 0.381) (layer "B.Cu") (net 10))
 (segment (start 143.32775 80.63) (end 142.98 80.63) (width 0.381) (layer "B.Cu") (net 10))
 (segment (start 156.1155 89.8555) (end 155 88.74) (width 0.381) (layer "B.Cu") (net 10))
 (segment (start 156.1105 96.4355) (end 156.1105 97.697804) (width 0.381) (layer "B.Cu") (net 10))
 (segment (start 156.1155 94.2495) (end 156.1155 89.8555) (width 0.381) (layer "B.Cu") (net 10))
 (segment (start 155 85.73) (end 148.08 78.81) (width 0.381) (layer "B.Cu") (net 10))
 (segment (start 134.7145 83.1555) (end 134.7145 85.5855) (width 0.381) (layer "B.Cu") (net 10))
 (segment (start 146.89 100.28) (end 146.99 100.38) (width 0.381) (layer "B.Cu") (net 10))
 (segment (start 139.74 80.7) (end 137.17 80.7) (width 0.381) (layer "B.Cu") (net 10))
 (segment (start 139.96 100.28) (end 146.89 100.28) (width 0.381) (layer "B.Cu") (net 10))
 (segment (start 155.02 95.345) (end 156.1155 94.2495) (width 0.381) (layer "B.Cu") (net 10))
 (segment (start 155.02 95.345) (end 156.1105 96.4355) (width 0.381) (layer "B.Cu") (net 10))
 (segment (start 142.98 80.63) (end 139.81 80.63) (width 0.381) (layer "B.Cu") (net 10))
 (segment (start 131.91 88.39) (end 135.68 92.16) (width 0.381) (layer "B.Cu") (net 10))
 (segment (start 139.81 80.63) (end 139.74 80.7) (width 0.381) (layer "B.Cu") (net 10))
 (segment (start 124.63 100.28) (end 138.06 100.28) (width 0.381) (layer "B.Cu") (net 12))
 (segment (start 115.96 91.61) (end 124.63 100.28) (width 0.381) (layer "B.Cu") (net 12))
 (segment (start 110.3714 115.5114) (end 108.96 114.1) (width 0.25) (layer "F.Cu") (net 8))
 (segment (start 128.43 114.1025) (end 127.0211 115.5114) (width 0.25) (layer "F.Cu") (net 8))
 (segment (start 127.0211 115.5114) (end 110.3714 115.5114) (width 0.25) (layer "F.Cu") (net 8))
 (segment (start 126.335 112.2275) (end 122.75 108.6425) (width 0.25) (layer "F.Cu") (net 3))
 (segment (start 128.43 112.2275) (end 126.335 112.2275) (width 0.25) (layer "F.Cu") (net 3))
 (segment (start 115.96 88.81) (end 115.96 82.853893) (width 0.381) (layer "B.Cu") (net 45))
 (segment (start 120.92 77.893893) (end 120.92 77.69) (width 0.381) (layer "B.Cu") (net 45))
 (segment (start 115.96 82.853893) (end 120.92 77.893893) (width 0.381) (layer "B.Cu") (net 45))
 (segment (start 122.84 80.45) (end 122.44 80.85) (width 0.2) (layer "B.Cu") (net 43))
 (segment (start 122.84 79.76) (end 122.84 80.45) (width 0.2) (layer "B.Cu") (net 43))
 (segment (start 122.52 79.44) (end 122.84 79.76) (width 0.2) (layer "B.Cu") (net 43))
 (segment (start 123.46 82.82) (end 123.46 84.8875) (width 0.2) (layer "B.Cu") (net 43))
 (segment (start 122.52 77.69) (end 122.52 79.44) (width 0.2) (layer "B.Cu") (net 43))
 (segment (start 122.44 81.8) (end 123.46 82.82) (width 0.2) (layer "B.Cu") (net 43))
 (segment (start 122.44 80.85) (end 122.44 81.8) (width 0.2) (layer "B.Cu") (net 43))
 (segment (start 123.2525 86.7125) (end 129.5 92.96) (width 0.25) (layer "B.Cu") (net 16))
 (segment (start 129.5 92.96) (end 137.81 92.96) (width 0.25) (layer "B.Cu") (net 16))
 (segment (start 123.46 86.7125) (end 123.2525 86.7125) (width 0.25) (layer "B.Cu") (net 16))
 (segment (start 121.37 80.51) (end 121.79 80.93) (width 0.2) (layer "B.Cu") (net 42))
 (segment (start 121.79 81.83) (end 120.65 82.97) (width 0.2) (layer "B.Cu") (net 42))
 (segment (start 120.65 82.97) (end 120.65 84.9175) (width 0.2) (layer "B.Cu") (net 42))
 (segment (start 121.72 77.69) (end 121.72 79.43) (width 0.2) (layer "B.Cu") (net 42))
 (segment (start 121.72 79.43) (end 121.37 79.78) (width 0.2) (layer "B.Cu") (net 42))
 (segment (start 121.37 79.78) (end 121.37 80.51) (width 0.2) (layer "B.Cu") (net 42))
 (segment (start 121.79 80.93) (end 121.79 81.83) (width 0.2) (layer "B.Cu") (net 42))
 (segment (start 127.6675 93.76) (end 137.81 93.76) (width 0.25) (layer "B.Cu") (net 15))
 (segment (start 120.65 86.7425) (end 127.6675 93.76) (width 0.25) (layer "B.Cu") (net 15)))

